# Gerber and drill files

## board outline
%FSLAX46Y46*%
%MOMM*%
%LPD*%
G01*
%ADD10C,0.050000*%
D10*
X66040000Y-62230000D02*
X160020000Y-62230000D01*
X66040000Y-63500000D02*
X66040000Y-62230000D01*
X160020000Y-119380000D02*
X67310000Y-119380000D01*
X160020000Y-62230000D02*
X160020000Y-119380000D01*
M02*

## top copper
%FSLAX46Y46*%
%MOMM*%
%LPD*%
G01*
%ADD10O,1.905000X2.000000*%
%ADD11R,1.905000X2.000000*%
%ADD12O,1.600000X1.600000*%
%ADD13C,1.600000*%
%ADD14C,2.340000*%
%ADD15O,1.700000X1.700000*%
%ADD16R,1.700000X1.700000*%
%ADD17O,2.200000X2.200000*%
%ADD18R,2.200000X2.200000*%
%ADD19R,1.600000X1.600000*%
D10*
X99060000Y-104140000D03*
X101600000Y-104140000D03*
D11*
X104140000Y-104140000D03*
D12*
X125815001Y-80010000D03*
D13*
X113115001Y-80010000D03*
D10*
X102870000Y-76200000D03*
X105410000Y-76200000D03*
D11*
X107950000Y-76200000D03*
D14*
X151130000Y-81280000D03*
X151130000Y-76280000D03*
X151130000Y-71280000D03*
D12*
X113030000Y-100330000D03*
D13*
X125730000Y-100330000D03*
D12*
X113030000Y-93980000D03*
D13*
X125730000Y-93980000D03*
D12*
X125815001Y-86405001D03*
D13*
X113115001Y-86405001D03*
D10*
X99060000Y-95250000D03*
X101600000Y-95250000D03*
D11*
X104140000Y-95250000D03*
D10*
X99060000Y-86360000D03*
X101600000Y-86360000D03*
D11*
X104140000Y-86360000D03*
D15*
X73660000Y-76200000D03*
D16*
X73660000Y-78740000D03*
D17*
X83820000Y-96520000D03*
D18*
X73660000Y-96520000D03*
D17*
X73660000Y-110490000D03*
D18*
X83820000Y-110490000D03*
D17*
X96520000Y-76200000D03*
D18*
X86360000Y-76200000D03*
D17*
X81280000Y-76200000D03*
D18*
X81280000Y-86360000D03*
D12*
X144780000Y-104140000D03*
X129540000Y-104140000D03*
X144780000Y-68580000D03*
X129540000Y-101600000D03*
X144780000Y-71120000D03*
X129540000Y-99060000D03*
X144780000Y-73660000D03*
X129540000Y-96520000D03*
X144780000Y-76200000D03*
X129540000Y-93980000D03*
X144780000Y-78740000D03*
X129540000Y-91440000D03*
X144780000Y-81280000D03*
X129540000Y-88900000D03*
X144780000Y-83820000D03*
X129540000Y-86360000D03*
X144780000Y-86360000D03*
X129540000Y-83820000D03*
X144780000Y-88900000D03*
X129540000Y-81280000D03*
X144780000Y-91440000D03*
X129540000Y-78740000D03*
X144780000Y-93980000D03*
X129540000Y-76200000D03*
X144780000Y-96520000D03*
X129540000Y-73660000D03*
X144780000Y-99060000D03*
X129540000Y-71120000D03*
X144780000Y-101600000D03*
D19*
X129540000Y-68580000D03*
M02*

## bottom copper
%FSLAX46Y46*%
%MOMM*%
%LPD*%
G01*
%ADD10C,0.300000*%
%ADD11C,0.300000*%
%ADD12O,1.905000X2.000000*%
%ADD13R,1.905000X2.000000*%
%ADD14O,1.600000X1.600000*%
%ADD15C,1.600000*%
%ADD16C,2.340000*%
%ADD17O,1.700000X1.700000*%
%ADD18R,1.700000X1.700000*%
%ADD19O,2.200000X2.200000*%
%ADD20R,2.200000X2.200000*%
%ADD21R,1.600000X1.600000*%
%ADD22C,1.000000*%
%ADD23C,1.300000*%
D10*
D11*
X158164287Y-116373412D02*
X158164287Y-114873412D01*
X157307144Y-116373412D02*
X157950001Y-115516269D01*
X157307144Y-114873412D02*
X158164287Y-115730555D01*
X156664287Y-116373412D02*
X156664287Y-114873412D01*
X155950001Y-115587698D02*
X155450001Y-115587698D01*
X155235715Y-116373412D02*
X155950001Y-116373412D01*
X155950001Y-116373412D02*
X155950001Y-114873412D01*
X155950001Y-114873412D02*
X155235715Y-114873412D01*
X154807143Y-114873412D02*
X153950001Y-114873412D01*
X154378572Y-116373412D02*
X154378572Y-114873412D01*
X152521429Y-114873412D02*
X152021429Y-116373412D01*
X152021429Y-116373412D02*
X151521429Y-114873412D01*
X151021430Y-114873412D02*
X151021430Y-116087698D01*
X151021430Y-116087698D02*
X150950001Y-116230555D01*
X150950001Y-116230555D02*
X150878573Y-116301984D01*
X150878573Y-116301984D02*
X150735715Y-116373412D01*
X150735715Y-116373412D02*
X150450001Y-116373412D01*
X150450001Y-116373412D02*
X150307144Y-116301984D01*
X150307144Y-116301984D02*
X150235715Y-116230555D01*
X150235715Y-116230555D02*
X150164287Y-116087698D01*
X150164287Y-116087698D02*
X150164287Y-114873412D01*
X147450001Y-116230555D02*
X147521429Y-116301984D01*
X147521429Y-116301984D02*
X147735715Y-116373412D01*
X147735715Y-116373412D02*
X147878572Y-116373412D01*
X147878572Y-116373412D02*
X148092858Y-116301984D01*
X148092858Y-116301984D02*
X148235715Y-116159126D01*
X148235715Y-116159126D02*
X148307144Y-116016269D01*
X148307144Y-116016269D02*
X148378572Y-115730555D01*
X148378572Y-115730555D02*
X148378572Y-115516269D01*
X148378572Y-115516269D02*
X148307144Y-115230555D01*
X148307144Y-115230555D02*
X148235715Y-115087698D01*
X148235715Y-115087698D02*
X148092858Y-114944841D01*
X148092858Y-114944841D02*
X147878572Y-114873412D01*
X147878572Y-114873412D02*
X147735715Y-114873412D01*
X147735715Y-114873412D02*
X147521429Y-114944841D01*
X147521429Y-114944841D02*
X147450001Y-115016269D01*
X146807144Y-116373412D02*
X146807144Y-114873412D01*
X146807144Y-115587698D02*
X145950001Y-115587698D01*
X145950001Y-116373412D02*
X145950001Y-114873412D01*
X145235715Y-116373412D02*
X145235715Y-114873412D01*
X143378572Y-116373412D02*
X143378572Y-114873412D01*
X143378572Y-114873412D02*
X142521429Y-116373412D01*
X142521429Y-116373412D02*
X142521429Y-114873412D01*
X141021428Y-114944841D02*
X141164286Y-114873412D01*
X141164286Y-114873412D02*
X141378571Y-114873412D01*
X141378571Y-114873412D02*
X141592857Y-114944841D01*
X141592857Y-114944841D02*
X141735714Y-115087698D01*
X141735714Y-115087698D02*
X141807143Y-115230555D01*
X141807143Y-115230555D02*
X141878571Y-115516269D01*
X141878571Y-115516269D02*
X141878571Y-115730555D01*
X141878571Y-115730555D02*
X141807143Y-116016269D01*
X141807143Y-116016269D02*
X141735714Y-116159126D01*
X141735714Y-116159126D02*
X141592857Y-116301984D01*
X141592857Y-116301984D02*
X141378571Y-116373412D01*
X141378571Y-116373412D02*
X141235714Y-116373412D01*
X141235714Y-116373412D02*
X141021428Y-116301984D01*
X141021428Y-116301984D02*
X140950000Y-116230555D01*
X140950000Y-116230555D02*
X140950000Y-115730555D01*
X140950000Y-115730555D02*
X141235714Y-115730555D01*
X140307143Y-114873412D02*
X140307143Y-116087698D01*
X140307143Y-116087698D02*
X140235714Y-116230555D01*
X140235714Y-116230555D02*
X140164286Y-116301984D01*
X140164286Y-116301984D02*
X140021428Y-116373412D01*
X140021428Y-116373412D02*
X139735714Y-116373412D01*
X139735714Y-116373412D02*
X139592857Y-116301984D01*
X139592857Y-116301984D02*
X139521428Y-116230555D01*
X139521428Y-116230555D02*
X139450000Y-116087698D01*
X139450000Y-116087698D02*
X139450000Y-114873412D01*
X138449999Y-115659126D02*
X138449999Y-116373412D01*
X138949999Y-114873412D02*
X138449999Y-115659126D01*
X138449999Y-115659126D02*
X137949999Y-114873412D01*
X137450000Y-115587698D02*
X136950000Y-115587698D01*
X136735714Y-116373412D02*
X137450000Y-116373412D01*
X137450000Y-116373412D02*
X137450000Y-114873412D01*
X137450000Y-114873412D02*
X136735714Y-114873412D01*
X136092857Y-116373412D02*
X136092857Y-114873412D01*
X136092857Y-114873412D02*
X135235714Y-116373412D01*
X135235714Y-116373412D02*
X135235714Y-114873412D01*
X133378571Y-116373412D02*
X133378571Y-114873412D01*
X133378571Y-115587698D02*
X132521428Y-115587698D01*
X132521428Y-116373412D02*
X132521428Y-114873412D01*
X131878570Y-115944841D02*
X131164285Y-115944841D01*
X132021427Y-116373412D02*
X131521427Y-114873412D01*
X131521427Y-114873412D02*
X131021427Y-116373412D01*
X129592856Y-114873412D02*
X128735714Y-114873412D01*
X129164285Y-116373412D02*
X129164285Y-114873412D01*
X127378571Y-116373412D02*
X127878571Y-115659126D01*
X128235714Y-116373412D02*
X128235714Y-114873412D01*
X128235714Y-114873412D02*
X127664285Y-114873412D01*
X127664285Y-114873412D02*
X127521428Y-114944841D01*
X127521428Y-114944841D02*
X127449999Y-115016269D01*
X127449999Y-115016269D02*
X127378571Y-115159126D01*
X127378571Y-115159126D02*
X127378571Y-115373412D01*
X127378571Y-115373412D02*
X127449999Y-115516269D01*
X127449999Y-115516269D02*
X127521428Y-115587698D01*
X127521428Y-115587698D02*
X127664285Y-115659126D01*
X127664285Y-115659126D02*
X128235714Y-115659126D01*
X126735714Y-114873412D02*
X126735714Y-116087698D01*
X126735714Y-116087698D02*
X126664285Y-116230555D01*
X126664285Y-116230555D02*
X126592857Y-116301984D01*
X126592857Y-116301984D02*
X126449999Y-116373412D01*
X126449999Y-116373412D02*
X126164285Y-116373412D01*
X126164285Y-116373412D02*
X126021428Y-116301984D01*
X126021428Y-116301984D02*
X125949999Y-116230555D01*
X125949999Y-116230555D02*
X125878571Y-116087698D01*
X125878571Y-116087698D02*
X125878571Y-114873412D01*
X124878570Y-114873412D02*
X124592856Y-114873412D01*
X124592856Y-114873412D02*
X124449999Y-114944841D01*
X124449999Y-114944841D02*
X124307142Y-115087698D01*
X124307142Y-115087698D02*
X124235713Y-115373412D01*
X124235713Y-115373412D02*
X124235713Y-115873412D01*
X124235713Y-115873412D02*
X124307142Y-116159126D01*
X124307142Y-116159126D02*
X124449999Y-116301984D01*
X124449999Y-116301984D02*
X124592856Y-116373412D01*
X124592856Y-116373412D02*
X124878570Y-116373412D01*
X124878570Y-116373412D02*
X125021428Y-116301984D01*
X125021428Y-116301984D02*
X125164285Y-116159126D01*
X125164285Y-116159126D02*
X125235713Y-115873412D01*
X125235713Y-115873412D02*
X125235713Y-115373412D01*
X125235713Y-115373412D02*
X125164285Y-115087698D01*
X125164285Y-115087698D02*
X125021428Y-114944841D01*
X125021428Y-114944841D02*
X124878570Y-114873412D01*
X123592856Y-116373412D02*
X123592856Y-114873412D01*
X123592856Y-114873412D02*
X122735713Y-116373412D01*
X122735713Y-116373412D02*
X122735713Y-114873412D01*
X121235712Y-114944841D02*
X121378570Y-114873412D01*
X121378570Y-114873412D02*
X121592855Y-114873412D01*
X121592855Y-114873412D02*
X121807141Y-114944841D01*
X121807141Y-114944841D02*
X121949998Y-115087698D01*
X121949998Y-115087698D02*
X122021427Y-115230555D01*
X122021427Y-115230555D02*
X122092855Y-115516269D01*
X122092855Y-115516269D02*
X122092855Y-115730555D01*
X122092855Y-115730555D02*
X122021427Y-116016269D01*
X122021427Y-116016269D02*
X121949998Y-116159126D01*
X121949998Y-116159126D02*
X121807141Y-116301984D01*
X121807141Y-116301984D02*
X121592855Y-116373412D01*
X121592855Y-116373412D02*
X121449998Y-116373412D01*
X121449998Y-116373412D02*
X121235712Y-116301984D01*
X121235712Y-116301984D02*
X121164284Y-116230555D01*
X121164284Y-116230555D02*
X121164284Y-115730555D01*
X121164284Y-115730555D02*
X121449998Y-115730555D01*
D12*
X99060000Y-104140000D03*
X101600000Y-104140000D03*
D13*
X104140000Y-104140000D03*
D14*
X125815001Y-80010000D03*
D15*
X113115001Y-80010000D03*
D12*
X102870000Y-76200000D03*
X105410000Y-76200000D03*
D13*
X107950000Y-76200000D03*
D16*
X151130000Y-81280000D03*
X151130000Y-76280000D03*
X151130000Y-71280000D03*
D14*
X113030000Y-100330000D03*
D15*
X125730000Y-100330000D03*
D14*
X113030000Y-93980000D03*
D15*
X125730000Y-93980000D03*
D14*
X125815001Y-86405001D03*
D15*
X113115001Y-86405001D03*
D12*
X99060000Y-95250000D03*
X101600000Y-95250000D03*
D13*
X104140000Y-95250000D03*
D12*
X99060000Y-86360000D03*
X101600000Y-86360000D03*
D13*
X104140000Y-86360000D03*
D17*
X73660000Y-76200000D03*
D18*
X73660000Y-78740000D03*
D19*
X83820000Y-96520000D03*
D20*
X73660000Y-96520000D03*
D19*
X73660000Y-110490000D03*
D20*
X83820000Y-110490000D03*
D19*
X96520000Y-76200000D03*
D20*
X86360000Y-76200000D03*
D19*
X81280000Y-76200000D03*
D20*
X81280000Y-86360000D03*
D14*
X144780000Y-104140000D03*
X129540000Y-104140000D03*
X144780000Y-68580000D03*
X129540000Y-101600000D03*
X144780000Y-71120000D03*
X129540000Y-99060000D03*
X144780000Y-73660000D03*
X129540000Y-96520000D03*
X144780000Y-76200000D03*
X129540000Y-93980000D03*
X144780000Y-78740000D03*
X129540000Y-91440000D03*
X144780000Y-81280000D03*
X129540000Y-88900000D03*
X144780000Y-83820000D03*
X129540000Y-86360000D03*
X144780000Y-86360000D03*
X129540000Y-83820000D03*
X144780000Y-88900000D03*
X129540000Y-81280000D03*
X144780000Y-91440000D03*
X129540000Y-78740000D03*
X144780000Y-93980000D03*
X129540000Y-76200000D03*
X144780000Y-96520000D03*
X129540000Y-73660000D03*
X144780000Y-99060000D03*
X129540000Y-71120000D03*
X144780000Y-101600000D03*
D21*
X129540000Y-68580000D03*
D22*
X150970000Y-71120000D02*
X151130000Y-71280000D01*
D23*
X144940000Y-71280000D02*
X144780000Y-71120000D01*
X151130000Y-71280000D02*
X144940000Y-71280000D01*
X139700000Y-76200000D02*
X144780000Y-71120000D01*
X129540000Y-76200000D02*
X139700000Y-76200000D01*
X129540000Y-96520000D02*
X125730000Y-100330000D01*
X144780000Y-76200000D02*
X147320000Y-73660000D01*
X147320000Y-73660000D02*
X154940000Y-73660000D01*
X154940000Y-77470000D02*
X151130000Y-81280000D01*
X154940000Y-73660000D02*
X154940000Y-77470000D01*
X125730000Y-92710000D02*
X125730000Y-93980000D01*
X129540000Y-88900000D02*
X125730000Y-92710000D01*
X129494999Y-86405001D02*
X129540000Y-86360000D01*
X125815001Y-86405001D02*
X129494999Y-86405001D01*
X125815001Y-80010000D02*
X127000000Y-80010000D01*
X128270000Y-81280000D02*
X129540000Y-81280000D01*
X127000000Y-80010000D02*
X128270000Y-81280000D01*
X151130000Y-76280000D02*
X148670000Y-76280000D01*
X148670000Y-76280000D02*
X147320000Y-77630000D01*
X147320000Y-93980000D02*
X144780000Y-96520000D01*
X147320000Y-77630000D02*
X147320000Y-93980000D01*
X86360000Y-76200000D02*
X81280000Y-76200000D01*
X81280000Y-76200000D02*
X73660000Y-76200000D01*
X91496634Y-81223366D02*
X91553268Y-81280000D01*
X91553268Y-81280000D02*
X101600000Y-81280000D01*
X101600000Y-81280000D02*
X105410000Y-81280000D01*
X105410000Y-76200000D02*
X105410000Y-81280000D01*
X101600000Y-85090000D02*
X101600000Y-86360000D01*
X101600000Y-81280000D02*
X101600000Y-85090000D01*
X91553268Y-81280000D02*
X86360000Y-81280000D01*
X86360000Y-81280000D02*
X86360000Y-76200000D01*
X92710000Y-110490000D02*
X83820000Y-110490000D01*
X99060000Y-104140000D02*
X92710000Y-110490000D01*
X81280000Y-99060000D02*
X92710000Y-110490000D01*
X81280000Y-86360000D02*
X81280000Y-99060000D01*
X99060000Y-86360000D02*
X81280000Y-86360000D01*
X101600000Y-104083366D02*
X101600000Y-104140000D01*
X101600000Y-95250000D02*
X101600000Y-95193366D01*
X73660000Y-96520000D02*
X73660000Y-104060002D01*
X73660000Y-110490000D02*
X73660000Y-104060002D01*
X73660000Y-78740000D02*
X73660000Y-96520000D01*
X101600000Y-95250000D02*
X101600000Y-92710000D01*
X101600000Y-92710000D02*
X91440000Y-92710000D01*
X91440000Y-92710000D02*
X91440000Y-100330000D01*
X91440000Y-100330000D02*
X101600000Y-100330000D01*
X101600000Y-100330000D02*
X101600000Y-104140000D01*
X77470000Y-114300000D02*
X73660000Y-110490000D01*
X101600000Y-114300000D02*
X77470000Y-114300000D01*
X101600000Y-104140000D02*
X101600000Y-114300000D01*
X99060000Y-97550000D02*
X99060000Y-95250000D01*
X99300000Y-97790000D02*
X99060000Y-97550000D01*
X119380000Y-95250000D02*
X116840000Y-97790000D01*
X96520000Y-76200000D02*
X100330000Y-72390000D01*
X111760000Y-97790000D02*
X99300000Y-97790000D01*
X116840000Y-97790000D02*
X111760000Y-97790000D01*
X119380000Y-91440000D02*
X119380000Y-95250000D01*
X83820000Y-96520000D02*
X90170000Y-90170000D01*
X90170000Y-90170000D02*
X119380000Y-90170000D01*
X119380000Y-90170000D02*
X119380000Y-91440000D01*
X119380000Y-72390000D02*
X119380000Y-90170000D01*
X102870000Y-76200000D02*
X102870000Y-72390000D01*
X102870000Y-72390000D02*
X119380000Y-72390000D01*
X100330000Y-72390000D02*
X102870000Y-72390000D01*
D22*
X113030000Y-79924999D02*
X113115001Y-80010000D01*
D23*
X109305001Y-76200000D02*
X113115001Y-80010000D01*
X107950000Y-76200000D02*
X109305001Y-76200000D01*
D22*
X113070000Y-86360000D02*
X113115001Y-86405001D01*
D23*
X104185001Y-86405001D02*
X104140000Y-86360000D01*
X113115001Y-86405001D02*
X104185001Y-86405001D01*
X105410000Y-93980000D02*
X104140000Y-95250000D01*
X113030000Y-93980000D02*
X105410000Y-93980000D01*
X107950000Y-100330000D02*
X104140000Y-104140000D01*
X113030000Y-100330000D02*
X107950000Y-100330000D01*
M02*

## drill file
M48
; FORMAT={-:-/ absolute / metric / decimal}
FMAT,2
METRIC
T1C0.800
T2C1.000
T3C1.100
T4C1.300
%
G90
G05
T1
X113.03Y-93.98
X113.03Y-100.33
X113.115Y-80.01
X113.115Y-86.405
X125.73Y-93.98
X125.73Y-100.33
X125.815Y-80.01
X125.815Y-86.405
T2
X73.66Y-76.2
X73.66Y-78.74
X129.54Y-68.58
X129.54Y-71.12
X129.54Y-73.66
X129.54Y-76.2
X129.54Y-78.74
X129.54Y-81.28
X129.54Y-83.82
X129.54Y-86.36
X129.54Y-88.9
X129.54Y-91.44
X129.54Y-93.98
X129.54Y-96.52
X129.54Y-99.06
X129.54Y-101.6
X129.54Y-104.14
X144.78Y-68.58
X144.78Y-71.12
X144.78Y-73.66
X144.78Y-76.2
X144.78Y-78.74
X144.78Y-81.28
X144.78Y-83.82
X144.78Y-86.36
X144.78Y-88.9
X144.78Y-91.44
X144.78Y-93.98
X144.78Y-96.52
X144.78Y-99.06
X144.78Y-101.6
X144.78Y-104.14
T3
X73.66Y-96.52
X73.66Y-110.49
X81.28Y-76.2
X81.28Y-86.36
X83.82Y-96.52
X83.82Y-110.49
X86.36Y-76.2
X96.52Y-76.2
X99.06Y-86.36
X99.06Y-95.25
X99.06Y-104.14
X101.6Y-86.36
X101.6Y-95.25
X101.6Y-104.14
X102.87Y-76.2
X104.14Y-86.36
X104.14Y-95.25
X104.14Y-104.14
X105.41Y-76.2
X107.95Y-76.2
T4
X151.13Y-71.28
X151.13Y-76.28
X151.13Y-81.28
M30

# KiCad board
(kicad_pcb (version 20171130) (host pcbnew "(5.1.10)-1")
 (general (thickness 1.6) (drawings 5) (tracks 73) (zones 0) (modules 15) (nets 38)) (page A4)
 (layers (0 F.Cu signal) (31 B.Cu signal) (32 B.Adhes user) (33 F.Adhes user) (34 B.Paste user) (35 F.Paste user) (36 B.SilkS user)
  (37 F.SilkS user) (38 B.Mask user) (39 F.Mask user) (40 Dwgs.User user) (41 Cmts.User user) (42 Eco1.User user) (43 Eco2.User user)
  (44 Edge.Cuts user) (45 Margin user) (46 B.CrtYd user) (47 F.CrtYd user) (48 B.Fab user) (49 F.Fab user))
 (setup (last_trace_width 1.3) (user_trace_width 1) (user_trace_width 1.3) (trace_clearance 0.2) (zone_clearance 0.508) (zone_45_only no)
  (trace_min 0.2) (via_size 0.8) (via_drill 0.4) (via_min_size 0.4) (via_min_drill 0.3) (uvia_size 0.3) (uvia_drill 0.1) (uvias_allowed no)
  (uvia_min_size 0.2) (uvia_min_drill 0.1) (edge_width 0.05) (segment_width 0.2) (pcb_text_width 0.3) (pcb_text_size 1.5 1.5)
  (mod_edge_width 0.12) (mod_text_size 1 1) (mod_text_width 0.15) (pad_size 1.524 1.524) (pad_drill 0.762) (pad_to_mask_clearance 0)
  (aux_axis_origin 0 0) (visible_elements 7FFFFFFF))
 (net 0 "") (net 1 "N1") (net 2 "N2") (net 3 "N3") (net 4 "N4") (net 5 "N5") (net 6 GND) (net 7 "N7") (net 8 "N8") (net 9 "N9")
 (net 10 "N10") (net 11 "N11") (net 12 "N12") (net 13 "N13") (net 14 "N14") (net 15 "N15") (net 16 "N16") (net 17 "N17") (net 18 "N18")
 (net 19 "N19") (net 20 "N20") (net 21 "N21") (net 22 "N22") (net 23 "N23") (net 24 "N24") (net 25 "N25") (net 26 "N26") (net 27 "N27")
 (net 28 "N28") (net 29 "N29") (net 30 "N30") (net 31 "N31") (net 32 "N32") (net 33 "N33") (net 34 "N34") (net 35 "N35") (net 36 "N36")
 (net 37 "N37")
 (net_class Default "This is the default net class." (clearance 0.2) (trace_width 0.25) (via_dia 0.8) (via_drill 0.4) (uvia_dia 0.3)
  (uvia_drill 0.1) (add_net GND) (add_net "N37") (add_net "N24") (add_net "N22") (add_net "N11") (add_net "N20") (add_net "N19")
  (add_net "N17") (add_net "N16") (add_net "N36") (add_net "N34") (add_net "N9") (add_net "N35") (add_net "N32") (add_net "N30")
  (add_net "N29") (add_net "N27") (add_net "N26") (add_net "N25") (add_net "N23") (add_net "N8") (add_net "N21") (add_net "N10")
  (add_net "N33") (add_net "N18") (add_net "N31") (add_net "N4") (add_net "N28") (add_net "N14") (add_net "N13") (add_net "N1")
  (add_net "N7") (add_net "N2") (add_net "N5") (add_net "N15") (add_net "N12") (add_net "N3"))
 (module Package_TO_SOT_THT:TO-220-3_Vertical (layer F.Cu) (at 104.14 104.14 180)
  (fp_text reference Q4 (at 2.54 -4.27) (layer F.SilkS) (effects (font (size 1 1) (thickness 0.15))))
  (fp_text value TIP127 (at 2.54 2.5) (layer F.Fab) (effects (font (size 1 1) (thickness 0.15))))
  (pad 3 thru_hole oval (at 5.08 0 180) (size 1.905 2) (drill 1.1) (layers *.Cu *.Mask) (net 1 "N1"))
  (pad 2 thru_hole oval (at 2.54 0 180) (size 1.905 2) (drill 1.1) (layers *.Cu *.Mask) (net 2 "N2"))
  (pad 1 thru_hole rect (at 0 0 180) (size 1.905 2) (drill 1.1) (layers *.Cu *.Mask) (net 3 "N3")))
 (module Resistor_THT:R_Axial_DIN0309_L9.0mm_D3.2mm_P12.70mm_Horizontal (layer F.Cu) (at 113.115001 80.01)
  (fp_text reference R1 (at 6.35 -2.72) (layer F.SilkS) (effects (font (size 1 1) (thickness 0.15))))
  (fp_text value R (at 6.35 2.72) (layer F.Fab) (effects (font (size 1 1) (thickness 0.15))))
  (pad 2 thru_hole oval (at 12.7 0) (size 1.6 1.6) (drill 0.8) (layers *.Cu *.Mask) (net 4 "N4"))
  (pad 1 thru_hole circle (at 0 0) (size 1.6 1.6) (drill 0.8) (layers *.Cu *.Mask) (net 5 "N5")))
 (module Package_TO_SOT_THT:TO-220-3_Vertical (layer F.Cu) (at 107.95 76.2 180)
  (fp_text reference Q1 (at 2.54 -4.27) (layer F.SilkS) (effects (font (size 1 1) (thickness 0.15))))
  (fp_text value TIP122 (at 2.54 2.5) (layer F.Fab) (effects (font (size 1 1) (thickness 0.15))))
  (pad 3 thru_hole oval (at 5.08 0 180) (size 1.905 2) (drill 1.1) (layers *.Cu *.Mask) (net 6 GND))
  (pad 2 thru_hole oval (at 2.54 0 180) (size 1.905 2) (drill 1.1) (layers *.Cu *.Mask) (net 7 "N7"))
  (pad 1 thru_hole rect (at 0 0 180) (size 1.905 2) (drill 1.1) (layers *.Cu *.Mask) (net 5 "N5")))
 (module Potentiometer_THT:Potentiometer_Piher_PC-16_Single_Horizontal (layer F.Cu) (at 151.13 81.28)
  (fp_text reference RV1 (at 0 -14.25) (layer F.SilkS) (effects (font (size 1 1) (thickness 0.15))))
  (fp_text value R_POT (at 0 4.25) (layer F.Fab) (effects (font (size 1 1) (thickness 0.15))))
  (pad 1 thru_hole circle (at 0 0) (size 2.34 2.34) (drill 1.3) (layers *.Cu *.Mask) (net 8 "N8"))
  (pad 2 thru_hole circle (at 0 -5) (size 2.34 2.34) (drill 1.3) (layers *.Cu *.Mask) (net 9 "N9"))
  (pad 3 thru_hole circle (at 0 -10) (size 2.34 2.34) (drill 1.3) (layers *.Cu *.Mask) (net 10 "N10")))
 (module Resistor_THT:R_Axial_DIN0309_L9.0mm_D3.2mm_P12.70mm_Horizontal (layer F.Cu) (at 125.73 100.33 180)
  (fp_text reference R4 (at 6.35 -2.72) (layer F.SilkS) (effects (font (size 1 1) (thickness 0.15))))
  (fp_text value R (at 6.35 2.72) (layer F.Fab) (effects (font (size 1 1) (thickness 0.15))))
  (pad 2 thru_hole oval (at 12.7 0 180) (size 1.6 1.6) (drill 0.8) (layers *.Cu *.Mask) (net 3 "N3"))
  (pad 1 thru_hole circle (at 0 0 180) (size 1.6 1.6) (drill 0.8) (layers *.Cu *.Mask) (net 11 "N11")))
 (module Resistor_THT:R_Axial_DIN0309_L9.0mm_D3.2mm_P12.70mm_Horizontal (layer F.Cu) (at 125.73 93.98 180)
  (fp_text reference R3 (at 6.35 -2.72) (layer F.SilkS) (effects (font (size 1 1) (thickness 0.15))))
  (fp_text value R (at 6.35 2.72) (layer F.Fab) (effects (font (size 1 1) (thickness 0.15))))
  (pad 2 thru_hole oval (at 12.7 0 180) (size 1.6 1.6) (drill 0.8) (layers *.Cu *.Mask) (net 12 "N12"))
  (pad 1 thru_hole circle (at 0 0 180) (size 1.6 1.6) (drill 0.8) (layers *.Cu *.Mask) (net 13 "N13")))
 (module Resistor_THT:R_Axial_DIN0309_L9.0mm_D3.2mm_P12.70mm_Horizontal (layer F.Cu) (at 113.115001 86.405001)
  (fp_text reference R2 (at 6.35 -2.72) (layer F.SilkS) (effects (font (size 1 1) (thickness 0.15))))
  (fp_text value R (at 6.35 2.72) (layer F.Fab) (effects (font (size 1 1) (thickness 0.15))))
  (pad 2 thru_hole oval (at 12.7 0) (size 1.6 1.6) (drill 0.8) (layers *.Cu *.Mask) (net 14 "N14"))
  (pad 1 thru_hole circle (at 0 0) (size 1.6 1.6) (drill 0.8) (layers *.Cu *.Mask) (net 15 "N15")))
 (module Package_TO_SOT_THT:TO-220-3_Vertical (layer F.Cu) (at 104.14 95.25 180)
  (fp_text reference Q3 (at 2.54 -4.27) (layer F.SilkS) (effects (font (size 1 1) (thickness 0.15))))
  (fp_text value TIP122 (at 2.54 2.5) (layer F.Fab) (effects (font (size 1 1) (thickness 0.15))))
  (pad 3 thru_hole oval (at 5.08 0 180) (size 1.905 2) (drill 1.1) (layers *.Cu *.Mask) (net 6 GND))
  (pad 2 thru_hole oval (at 2.54 0 180) (size 1.905 2) (drill 1.1) (layers *.Cu *.Mask) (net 2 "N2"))
  (pad 1 thru_hole rect (at 0 0 180) (size 1.905 2) (drill 1.1) (layers *.Cu *.Mask) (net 12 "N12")))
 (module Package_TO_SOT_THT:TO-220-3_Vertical (layer F.Cu) (at 104.14 86.36 180)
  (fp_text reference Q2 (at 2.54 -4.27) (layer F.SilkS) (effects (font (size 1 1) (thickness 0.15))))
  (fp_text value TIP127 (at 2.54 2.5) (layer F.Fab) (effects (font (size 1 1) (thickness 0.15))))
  (pad 3 thru_hole oval (at 5.08 0 180) (size 1.905 2) (drill 1.1) (layers *.Cu *.Mask) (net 1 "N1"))
  (pad 2 thru_hole oval (at 2.54 0 180) (size 1.905 2) (drill 1.1) (layers *.Cu *.Mask) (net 7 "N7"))
  (pad 1 thru_hole rect (at 0 0 180) (size 1.905 2) (drill 1.1) (layers *.Cu *.Mask) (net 15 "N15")))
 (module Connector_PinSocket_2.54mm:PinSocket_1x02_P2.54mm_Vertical (layer F.Cu) (at 73.66 78.74 180)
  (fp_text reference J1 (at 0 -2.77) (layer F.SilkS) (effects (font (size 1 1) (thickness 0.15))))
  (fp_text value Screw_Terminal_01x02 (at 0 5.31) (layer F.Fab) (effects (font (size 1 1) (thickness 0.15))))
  (pad 2 thru_hole oval (at 0 2.54 180) (size 1.7 1.7) (drill 1) (layers *.Cu *.Mask) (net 7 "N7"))
  (pad 1 thru_hole rect (at 0 0 180) (size 1.7 1.7) (drill 1) (layers *.Cu *.Mask) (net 2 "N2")))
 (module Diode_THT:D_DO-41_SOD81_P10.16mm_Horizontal (layer F.Cu) (at 73.66 96.52)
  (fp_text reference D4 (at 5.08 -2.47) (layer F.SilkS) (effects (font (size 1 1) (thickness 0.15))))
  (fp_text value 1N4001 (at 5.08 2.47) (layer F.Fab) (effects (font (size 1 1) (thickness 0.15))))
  (pad 2 thru_hole oval (at 10.16 0) (size 2.2 2.2) (drill 1.1) (layers *.Cu *.Mask) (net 6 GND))
  (pad 1 thru_hole rect (at 0 0) (size 2.2 2.2) (drill 1.1) (layers *.Cu *.Mask) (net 2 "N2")))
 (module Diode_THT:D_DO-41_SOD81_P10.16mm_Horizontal (layer F.Cu) (at 83.82 110.49 180)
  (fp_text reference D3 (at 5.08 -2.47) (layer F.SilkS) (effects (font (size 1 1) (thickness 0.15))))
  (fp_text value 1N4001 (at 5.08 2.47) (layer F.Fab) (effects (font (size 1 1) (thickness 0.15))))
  (pad 2 thru_hole oval (at 10.16 0 180) (size 2.2 2.2) (drill 1.1) (layers *.Cu *.Mask) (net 2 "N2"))
  (pad 1 thru_hole rect (at 0 0 180) (size 2.2 2.2) (drill 1.1) (layers *.Cu *.Mask) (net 1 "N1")))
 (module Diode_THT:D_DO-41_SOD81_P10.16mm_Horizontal (layer F.Cu) (at 86.36 76.2)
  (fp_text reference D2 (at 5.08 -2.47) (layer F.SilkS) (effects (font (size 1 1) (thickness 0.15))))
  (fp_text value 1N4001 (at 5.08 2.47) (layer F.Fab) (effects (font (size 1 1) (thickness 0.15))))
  (pad 2 thru_hole oval (at 10.16 0) (size 2.2 2.2) (drill 1.1) (layers *.Cu *.Mask) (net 6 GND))
  (pad 1 thru_hole rect (at 0 0) (size 2.2 2.2) (drill 1.1) (layers *.Cu *.Mask) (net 7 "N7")))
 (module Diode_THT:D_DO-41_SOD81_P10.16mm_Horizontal (layer F.Cu) (at 81.28 86.36 90)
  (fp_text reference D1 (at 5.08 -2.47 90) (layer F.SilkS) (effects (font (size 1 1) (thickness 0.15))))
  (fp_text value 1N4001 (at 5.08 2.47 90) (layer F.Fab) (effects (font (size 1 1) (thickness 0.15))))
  (pad 2 thru_hole oval (at 10.16 0 90) (size 2.2 2.2) (drill 1.1) (layers *.Cu *.Mask) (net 7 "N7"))
  (pad 1 thru_hole rect (at 0 0 90) (size 2.2 2.2) (drill 1.1) (layers *.Cu *.Mask) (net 1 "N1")))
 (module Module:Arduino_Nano (layer F.Cu) (at 129.54 68.58)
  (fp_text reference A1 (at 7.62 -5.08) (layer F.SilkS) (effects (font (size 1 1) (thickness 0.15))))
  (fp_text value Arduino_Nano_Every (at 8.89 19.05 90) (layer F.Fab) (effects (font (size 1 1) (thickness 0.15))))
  (pad 16 thru_hole oval (at 15.24 35.56) (size 1.6 1.6) (drill 1) (layers *.Cu *.Mask) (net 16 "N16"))
  (pad 15 thru_hole oval (at 0 35.56) (size 1.6 1.6) (drill 1) (layers *.Cu *.Mask) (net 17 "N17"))
  (pad 30 thru_hole oval (at 15.24 0) (size 1.6 1.6) (drill 1) (layers *.Cu *.Mask) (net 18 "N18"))
  (pad 14 thru_hole oval (at 0 33.02) (size 1.6 1.6) (drill 1) (layers *.Cu *.Mask) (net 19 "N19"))
  (pad 29 thru_hole oval (at 15.24 2.54) (size 1.6 1.6) (drill 1) (layers *.Cu *.Mask) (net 10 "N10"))
  (pad 13 thru_hole oval (at 0 30.48) (size 1.6 1.6) (drill 1) (layers *.Cu *.Mask) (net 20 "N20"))
  (pad 28 thru_hole oval (at 15.24 5.08) (size 1.6 1.6) (drill 1) (layers *.Cu *.Mask) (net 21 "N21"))
  (pad 12 thru_hole oval (at 0 27.94) (size 1.6 1.6) (drill 1) (layers *.Cu *.Mask) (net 11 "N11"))
  (pad 27 thru_hole oval (at 15.24 7.62) (size 1.6 1.6) (drill 1) (layers *.Cu *.Mask) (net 8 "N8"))
  (pad 11 thru_hole oval (at 0 25.4) (size 1.6 1.6) (drill 1) (layers *.Cu *.Mask) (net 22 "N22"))
  (pad 26 thru_hole oval (at 15.24 10.16) (size 1.6 1.6) (drill 1) (layers *.Cu *.Mask) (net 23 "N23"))
  (pad 10 thru_hole oval (at 0 22.86) (size 1.6 1.6) (drill 1) (layers *.Cu *.Mask) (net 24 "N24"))
  (pad 25 thru_hole oval (at 15.24 12.7) (size 1.6 1.6) (drill 1) (layers *.Cu *.Mask) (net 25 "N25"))
  (pad 9 thru_hole oval (at 0 20.32) (size 1.6 1.6) (drill 1) (layers *.Cu *.Mask) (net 13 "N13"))
  (pad 24 thru_hole oval (at 15.24 15.24) (size 1.6 1.6) (drill 1) (layers *.Cu *.Mask) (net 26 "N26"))
  (pad 8 thru_hole oval (at 0 17.78) (size 1.6 1.6) (drill 1) (layers *.Cu *.Mask) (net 14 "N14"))
  (pad 23 thru_hole oval (at 15.24 17.78) (size 1.6 1.6) (drill 1) (layers *.Cu *.Mask) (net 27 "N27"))
  (pad 7 thru_hole oval (at 0 15.24) (size 1.6 1.6) (drill 1) (layers *.Cu *.Mask) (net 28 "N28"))
  (pad 22 thru_hole oval (at 15.24 20.32) (size 1.6 1.6) (drill 1) (layers *.Cu *.Mask) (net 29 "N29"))
  (pad 6 thru_hole oval (at 0 12.7) (size 1.6 1.6) (drill 1) (layers *.Cu *.Mask) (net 4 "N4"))
  (pad 21 thru_hole oval (at 15.24 22.86) (size 1.6 1.6) (drill 1) (layers *.Cu *.Mask) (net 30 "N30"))
  (pad 5 thru_hole oval (at 0 10.16) (size 1.6 1.6) (drill 1) (layers *.Cu *.Mask) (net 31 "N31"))
  (pad 20 thru_hole oval (at 15.24 25.4) (size 1.6 1.6) (drill 1) (layers *.Cu *.Mask) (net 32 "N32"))
  (pad 4 thru_hole oval (at 0 7.62) (size 1.6 1.6) (drill 1) (layers *.Cu *.Mask) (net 10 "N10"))
  (pad 19 thru_hole oval (at 15.24 27.94) (size 1.6 1.6) (drill 1) (layers *.Cu *.Mask) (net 9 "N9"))
  (pad 3 thru_hole oval (at 0 5.08) (size 1.6 1.6) (drill 1) (layers *.Cu *.Mask) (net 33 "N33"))
  (pad 18 thru_hole oval (at 15.24 30.48) (size 1.6 1.6) (drill 1) (layers *.Cu *.Mask) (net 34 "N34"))
  (pad 2 thru_hole oval (at 0 2.54) (size 1.6 1.6) (drill 1) (layers *.Cu *.Mask) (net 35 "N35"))
  (pad 17 thru_hole oval (at 15.24 33.02) (size 1.6 1.6) (drill 1) (layers *.Cu *.Mask) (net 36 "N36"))
  (pad 1 thru_hole rect (at 0 0) (size 1.6 1.6) (drill 1) (layers *.Cu *.Mask) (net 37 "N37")))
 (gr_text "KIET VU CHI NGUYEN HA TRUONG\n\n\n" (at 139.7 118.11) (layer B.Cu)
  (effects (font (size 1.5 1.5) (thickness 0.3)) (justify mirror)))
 (gr_line (start 66.04 62.23) (end 160.02 62.23) (layer Edge.Cuts) (width 0.05))
 (gr_line (start 66.04 63.5) (end 66.04 62.23) (layer Edge.Cuts) (width 0.05))
 (gr_line (start 160.02 119.38) (end 67.31 119.38) (layer Edge.Cuts) (width 0.05))
 (gr_line (start 160.02 62.23) (end 160.02 119.38) (layer Edge.Cuts) (width 0.05))
 (segment (start 150.97 71.12) (end 151.13 71.28) (width 1) (layer B.Cu) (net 10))
 (segment (start 144.94 71.28) (end 144.78 71.12) (width 1.3) (layer B.Cu) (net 10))
 (segment (start 151.13 71.28) (end 144.94 71.28) (width 1.3) (layer B.Cu) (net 10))
 (segment (start 139.7 76.2) (end 144.78 71.12) (width 1.3) (layer B.Cu) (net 10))
 (segment (start 129.54 76.2) (end 139.7 76.2) (width 1.3) (layer B.Cu) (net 10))
 (segment (start 129.54 96.52) (end 125.73 100.33) (width 1.3) (layer B.Cu) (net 11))
 (segment (start 144.78 76.2) (end 147.32 73.66) (width 1.3) (layer B.Cu) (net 8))
 (segment (start 147.32 73.66) (end 154.94 73.66) (width 1.3) (layer B.Cu) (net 8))
 (segment (start 154.94 77.47) (end 151.13 81.28) (width 1.3) (layer B.Cu) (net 8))
 (segment (start 154.94 73.66) (end 154.94 77.47) (width 1.3) (layer B.Cu) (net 8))
 (segment (start 125.73 92.71) (end 125.73 93.98) (width 1.3) (layer B.Cu) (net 13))
 (segment (start 129.54 88.9) (end 125.73 92.71) (width 1.3) (layer B.Cu) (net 13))
 (segment (start 129.494999 86.405001) (end 129.54 86.36) (width 1.3) (layer B.Cu) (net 14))
 (segment (start 125.815001 86.405001) (end 129.494999 86.405001) (width 1.3) (layer B.Cu) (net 14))
 (segment (start 125.815001 80.01) (end 127 80.01) (width 1.3) (layer B.Cu) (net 4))
 (segment (start 128.27 81.28) (end 129.54 81.28) (width 1.3) (layer B.Cu) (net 4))
 (segment (start 127 80.01) (end 128.27 81.28) (width 1.3) (layer B.Cu) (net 4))
 (segment (start 151.13 76.28) (end 148.67 76.28) (width 1.3) (layer B.Cu) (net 9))
 (segment (start 148.67 76.28) (end 147.32 77.63) (width 1.3) (layer B.Cu) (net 9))
 (segment (start 147.32 93.98) (end 144.78 96.52) (width 1.3) (layer B.Cu) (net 9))
 (segment (start 147.32 77.63) (end 147.32 93.98) (width 1.3) (layer B.Cu) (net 9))
 (segment (start 86.36 76.2) (end 81.28 76.2) (width 1.3) (layer B.Cu) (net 7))
 (segment (start 81.28 76.2) (end 73.66 76.2) (width 1.3) (layer B.Cu) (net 7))
 (segment (start 91.496634 81.223366) (end 91.553268 81.28) (width 1.3) (layer B.Cu) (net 7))
 (segment (start 91.553268 81.28) (end 101.6 81.28) (width 1.3) (layer B.Cu) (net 7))
 (segment (start 101.6 81.28) (end 105.41 81.28) (width 1.3) (layer B.Cu) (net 7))
 (segment (start 105.41 76.2) (end 105.41 81.28) (width 1.3) (layer B.Cu) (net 7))
 (segment (start 101.6 85.09) (end 101.6 86.36) (width 1.3) (layer B.Cu) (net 7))
 (segment (start 101.6 81.28) (end 101.6 85.09) (width 1.3) (layer B.Cu) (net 7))
 (segment (start 91.553268 81.28) (end 86.36 81.28) (width 1.3) (layer B.Cu) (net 7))
 (segment (start 86.36 81.28) (end 86.36 76.2) (width 1.3) (layer B.Cu) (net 7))
 (segment (start 92.71 110.49) (end 83.82 110.49) (width 1.3) (layer B.Cu) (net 1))
 (segment (start 99.06 104.14) (end 92.71 110.49) (width 1.3) (layer B.Cu) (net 1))
 (segment (start 81.28 99.06) (end 92.71 110.49) (width 1.3) (layer B.Cu) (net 1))
 (segment (start 81.28 86.36) (end 81.28 99.06) (width 1.3) (layer B.Cu) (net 1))
 (segment (start 99.06 86.36) (end 81.28 86.36) (width 1.3) (layer B.Cu) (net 1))
 (segment (start 101.6 104.083366) (end 101.6 104.14) (width 1.3) (layer B.Cu) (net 2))
 (segment (start 101.6 95.25) (end 101.6 95.193366) (width 1.3) (layer B.Cu) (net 2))
 (segment (start 73.66 96.52) (end 73.66 104.060002) (width 1.3) (layer B.Cu) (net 2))
 (segment (start 73.66 110.49) (end 73.66 104.060002) (width 1.3) (layer B.Cu) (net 2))
 (segment (start 73.66 78.74) (end 73.66 96.52) (width 1.3) (layer B.Cu) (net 2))
 (segment (start 101.6 95.25) (end 101.6 92.71) (width 1.3) (layer B.Cu) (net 2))
 (segment (start 101.6 92.71) (end 91.44 92.71) (width 1.3) (layer B.Cu) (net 2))
 (segment (start 91.44 92.71) (end 91.44 100.33) (width 1.3) (layer B.Cu) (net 2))
 (segment (start 91.44 100.33) (end 101.6 100.33) (width 1.3) (layer B.Cu) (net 2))
 (segment (start 101.6 100.33) (end 101.6 104.14) (width 1.3) (layer B.Cu) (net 2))
 (segment (start 77.47 114.3) (end 73.66 110.49) (width 1.3) (layer B.Cu) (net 2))
 (segment (start 101.6 114.3) (end 77.47 114.3) (width 1.3) (layer B.Cu) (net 2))
 (segment (start 101.6 104.14) (end 101.6 114.3) (width 1.3) (layer B.Cu) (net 2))
 (segment (start 99.06 97.55) (end 99.06 95.25) (width 1.3) (layer B.Cu) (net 6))
 (segment (start 99.3 97.79) (end 99.06 97.55) (width 1.3) (layer B.Cu) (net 6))
 (segment (start 119.38 95.25) (end 116.84 97.79) (width 1.3) (layer B.Cu) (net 6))
 (segment (start 96.52 76.2) (end 100.33 72.39) (width 1.3) (layer B.Cu) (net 6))
 (segment (start 111.76 97.79) (end 99.3 97.79) (width 1.3) (layer B.Cu) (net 6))
 (segment (start 116.84 97.79) (end 111.76 97.79) (width 1.3) (layer B.Cu) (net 6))
 (segment (start 119.38 91.44) (end 119.38 95.25) (width 1.3) (layer B.Cu) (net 6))
 (segment (start 83.82 96.52) (end 90.17 90.17) (width 1.3) (layer B.Cu) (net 6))
 (segment (start 90.17 90.17) (end 119.38 90.17) (width 1.3) (layer B.Cu) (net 6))
 (segment (start 119.38 90.17) (end 119.38 91.44) (width 1.3) (layer B.Cu) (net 6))
 (segment (start 119.38 72.39) (end 119.38 90.17) (width 1.3) (layer B.Cu) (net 6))
 (segment (start 102.87 76.2) (end 102.87 72.39) (width 1.3) (layer B.Cu) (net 6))
 (segment (start 102.87 72.39) (end 119.38 72.39) (width 1.3) (layer B.Cu) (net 6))
 (segment (start 100.33 72.39) (end 102.87 72.39) (width 1.3) (layer B.Cu) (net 6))
 (segment (start 113.03 79.924999) (end 113.115001 80.01) (width 1) (layer B.Cu) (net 5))
 (segment (start 109.305001 76.2) (end 113.115001 80.01) (width 1.3) (layer B.Cu) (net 5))
 (segment (start 107.95 76.2) (end 109.305001 76.2) (width 1.3) (layer B.Cu) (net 5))
 (segment (start 113.07 86.36) (end 113.115001 86.405001) (width 1) (layer B.Cu) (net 15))
 (segment (start 104.185001 86.405001) (end 104.14 86.36) (width 1.3) (layer B.Cu) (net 15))
 (segment (start 113.115001 86.405001) (end 104.185001 86.405001) (width 1.3) (layer B.Cu) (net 15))
 (segment (start 105.41 93.98) (end 104.14 95.25) (width 1.3) (layer B.Cu) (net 12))
 (segment (start 113.03 93.98) (end 105.41 93.98) (width 1.3) (layer B.Cu) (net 12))
 (segment (start 107.95 100.33) (end 104.14 104.14) (width 1.3) (layer B.Cu) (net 3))
 (segment (start 113.03 100.33) (end 107.95 100.33) (width 1.3) (layer B.Cu) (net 3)))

